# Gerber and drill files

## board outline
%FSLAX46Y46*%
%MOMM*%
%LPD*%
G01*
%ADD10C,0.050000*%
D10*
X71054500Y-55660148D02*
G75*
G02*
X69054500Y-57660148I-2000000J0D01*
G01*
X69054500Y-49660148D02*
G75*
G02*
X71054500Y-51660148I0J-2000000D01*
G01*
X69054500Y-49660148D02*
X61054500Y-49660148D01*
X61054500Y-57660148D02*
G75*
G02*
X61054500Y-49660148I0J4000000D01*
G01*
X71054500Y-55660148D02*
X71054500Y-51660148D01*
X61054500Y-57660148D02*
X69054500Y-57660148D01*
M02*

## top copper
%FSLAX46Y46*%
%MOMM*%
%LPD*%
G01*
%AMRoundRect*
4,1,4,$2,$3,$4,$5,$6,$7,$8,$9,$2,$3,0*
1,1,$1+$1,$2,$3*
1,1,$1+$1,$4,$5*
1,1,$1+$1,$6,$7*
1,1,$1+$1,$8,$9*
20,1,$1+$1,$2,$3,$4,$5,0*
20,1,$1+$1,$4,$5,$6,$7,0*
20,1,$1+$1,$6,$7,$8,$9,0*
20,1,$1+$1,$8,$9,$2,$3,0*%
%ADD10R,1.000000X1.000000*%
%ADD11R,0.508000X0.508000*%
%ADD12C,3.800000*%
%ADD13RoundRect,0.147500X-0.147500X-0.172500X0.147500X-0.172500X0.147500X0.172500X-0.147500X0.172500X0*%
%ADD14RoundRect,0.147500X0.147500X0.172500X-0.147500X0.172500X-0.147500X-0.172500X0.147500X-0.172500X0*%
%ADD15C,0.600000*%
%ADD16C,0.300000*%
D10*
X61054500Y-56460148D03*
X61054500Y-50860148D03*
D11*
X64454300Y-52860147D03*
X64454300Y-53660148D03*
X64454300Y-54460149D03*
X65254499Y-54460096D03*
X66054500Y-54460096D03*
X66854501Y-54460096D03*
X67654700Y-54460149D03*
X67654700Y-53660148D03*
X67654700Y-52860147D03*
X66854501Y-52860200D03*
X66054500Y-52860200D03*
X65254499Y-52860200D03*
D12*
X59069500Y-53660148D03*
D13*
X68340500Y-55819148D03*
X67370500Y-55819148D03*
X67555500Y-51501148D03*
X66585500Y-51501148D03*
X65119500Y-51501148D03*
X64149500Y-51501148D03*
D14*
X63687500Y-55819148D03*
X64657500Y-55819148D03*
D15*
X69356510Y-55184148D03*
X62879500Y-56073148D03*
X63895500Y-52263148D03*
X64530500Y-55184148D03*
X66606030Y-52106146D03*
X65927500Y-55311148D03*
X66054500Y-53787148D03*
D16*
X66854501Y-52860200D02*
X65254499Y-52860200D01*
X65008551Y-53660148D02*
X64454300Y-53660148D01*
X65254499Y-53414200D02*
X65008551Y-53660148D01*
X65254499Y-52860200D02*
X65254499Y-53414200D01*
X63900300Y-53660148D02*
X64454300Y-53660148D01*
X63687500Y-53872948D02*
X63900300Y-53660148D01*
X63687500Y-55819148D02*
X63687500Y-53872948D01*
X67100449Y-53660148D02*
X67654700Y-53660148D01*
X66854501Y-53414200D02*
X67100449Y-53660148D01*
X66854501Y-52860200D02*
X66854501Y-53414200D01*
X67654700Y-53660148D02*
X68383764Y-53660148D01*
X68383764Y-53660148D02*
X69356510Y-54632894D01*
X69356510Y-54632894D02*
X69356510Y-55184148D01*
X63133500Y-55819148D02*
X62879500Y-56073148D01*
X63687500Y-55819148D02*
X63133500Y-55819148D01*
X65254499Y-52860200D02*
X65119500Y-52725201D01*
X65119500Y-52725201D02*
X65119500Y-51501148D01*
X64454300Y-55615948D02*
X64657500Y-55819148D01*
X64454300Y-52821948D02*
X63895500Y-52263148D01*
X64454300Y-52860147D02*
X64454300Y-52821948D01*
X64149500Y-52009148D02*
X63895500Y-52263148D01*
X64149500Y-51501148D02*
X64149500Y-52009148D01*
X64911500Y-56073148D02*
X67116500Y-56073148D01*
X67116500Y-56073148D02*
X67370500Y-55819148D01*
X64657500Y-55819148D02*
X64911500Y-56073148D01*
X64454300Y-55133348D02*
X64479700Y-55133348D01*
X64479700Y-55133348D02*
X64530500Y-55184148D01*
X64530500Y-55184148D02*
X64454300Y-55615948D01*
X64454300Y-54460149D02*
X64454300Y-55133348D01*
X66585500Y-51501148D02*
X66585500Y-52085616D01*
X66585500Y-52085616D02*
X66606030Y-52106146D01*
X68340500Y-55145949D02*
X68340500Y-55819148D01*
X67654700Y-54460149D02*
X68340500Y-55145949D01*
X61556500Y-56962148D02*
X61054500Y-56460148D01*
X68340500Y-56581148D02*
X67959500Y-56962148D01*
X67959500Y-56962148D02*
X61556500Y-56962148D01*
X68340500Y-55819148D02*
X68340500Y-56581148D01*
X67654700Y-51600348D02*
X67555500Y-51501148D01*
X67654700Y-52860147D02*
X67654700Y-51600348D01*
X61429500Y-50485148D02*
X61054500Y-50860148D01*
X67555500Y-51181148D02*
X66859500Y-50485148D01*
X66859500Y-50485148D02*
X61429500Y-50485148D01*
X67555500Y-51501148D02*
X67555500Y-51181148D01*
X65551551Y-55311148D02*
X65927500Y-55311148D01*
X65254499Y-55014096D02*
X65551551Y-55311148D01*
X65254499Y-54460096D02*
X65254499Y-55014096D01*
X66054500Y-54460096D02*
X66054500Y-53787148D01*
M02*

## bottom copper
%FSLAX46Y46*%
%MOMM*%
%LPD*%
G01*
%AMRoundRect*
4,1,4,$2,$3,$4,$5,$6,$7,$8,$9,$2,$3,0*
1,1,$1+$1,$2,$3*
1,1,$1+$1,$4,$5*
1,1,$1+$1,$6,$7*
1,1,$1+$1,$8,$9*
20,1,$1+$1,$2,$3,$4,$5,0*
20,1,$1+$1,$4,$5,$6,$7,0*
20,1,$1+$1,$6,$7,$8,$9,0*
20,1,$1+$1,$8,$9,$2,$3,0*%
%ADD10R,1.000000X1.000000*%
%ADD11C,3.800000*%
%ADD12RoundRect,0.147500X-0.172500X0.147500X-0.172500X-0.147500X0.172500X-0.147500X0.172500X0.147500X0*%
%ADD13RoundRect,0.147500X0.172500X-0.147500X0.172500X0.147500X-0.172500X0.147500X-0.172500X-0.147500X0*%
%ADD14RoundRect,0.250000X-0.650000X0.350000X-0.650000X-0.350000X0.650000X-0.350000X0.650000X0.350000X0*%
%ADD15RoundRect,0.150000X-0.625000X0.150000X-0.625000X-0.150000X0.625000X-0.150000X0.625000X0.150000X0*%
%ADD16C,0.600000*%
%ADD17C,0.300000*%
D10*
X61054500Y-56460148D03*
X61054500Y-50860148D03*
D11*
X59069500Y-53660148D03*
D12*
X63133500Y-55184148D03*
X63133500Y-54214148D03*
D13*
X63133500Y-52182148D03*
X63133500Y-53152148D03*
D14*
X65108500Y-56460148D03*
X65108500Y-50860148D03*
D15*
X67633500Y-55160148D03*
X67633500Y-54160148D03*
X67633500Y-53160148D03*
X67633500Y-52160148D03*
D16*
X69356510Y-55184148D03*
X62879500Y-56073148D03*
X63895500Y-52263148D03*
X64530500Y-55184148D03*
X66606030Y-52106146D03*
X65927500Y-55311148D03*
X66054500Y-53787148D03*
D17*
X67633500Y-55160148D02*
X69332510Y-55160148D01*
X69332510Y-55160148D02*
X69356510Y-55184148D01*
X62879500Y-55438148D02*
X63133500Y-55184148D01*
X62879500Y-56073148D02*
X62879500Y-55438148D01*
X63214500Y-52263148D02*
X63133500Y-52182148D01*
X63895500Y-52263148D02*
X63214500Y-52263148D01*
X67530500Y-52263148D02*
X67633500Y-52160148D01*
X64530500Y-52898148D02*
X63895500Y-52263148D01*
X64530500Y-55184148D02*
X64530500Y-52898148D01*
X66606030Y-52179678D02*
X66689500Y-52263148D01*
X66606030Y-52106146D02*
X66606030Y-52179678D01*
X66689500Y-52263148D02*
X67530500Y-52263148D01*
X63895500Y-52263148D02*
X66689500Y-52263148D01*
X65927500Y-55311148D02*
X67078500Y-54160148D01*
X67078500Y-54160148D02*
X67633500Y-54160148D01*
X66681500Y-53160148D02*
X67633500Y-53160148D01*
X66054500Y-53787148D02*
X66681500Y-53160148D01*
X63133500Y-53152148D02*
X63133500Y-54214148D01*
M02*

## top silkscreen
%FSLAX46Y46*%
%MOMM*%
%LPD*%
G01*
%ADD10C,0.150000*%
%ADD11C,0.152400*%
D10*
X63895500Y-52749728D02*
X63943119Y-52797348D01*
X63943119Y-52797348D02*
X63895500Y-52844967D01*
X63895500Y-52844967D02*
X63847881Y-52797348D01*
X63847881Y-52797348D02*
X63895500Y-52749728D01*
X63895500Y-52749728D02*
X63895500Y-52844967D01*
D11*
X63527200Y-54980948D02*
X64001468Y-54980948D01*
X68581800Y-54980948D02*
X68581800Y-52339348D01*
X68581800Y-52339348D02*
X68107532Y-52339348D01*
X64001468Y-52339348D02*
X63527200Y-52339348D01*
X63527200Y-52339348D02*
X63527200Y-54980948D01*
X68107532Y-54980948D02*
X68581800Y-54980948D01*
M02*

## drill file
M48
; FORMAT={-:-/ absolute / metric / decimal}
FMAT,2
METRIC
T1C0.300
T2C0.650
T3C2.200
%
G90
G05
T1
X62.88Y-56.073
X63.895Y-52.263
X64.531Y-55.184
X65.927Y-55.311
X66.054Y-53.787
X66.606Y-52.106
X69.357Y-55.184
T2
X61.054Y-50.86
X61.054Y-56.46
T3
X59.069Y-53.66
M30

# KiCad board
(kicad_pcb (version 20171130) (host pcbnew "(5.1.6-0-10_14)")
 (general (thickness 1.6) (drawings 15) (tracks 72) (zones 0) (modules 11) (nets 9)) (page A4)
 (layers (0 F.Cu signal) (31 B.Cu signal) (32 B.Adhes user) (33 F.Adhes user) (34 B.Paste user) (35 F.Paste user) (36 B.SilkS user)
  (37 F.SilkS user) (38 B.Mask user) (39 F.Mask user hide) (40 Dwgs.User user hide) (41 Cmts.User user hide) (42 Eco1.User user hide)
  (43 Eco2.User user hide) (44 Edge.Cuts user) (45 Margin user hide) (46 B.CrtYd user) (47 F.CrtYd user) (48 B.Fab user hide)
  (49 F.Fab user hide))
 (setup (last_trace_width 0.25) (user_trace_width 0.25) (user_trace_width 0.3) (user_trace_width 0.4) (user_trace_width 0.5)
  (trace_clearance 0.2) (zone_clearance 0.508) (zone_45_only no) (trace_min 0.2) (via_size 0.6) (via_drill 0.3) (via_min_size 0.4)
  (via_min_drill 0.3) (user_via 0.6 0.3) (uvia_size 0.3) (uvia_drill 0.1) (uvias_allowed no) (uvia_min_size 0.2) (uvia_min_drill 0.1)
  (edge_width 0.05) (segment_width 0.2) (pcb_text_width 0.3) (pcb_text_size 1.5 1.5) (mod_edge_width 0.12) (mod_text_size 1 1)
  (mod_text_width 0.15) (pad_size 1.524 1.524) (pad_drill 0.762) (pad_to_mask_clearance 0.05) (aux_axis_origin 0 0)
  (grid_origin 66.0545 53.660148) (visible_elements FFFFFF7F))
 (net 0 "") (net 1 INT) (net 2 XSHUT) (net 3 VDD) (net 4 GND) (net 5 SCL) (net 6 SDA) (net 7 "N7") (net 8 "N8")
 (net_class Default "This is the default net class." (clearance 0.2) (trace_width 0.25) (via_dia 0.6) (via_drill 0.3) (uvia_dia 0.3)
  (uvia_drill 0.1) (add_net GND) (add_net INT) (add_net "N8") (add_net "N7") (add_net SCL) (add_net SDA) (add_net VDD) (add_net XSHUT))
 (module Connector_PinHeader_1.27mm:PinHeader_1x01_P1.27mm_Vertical (layer F.Cu) (at 61.0545 56.460148)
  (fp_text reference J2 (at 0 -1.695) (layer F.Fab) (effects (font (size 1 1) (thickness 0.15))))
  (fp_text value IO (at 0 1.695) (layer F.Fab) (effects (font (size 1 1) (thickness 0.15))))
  (pad 1 thru_hole rect (at 0 0) (size 1 1) (drill 0.65) (layers *.Cu *.Mask) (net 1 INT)))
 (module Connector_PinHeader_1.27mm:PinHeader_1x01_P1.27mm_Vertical (layer F.Cu) (at 61.0545 50.860148 270)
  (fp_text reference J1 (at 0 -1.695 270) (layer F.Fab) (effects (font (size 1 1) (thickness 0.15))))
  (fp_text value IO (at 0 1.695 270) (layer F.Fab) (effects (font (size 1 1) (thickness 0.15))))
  (pad 1 thru_hole rect (at 0 0 270) (size 1 1) (drill 0.65) (layers *.Cu *.Mask) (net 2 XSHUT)))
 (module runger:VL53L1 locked (layer F.Cu) (at 66.0545 53.660148)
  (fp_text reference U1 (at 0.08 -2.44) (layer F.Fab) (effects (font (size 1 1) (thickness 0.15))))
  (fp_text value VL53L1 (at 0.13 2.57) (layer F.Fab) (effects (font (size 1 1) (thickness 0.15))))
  (fp_line (start -2.5273 1.3208) (end -2.053032 1.3208) (layer F.SilkS) (width 0.1524))
  (fp_line (start 2.5273 1.3208) (end 2.5273 -1.3208) (layer F.SilkS) (width 0.1524))
  (fp_line (start 2.5273 -1.3208) (end 2.053032 -1.3208) (layer F.SilkS) (width 0.1524))
  (fp_line (start -2.053032 -1.3208) (end -2.5273 -1.3208) (layer F.SilkS) (width 0.1524))
  (fp_line (start -2.5273 -1.3208) (end -2.5273 1.3208) (layer F.SilkS) (width 0.1524))
  (fp_line (start 2.053032 1.3208) (end 2.5273 1.3208) (layer F.SilkS) (width 0.1524))
  (pad 1 smd rect (at -1.6002 -0.800001 90) (size 0.508 0.508) (layers F.Cu F.Paste F.Mask) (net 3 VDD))
  (pad 12 smd rect (at -1.6002 0 90) (size 0.508 0.508) (layers F.Cu F.Paste F.Mask) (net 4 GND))
  (pad 11 smd rect (at -1.6002 0.800001 90) (size 0.508 0.508) (layers F.Cu F.Paste F.Mask) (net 3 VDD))
  (pad 10 smd rect (at -0.800001 0.799948) (size 0.508 0.508) (layers F.Cu F.Paste F.Mask) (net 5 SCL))
  (pad 9 smd rect (at 0 0.799948) (size 0.508 0.508) (layers F.Cu F.Paste F.Mask) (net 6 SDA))
  (pad 8 smd rect (at 0.800001 0.799948) (size 0.508 0.508) (layers F.Cu F.Paste F.Mask) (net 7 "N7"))
  (pad 7 smd rect (at 1.6002 0.800001 90) (size 0.508 0.508) (layers F.Cu F.Paste F.Mask) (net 1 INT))
  (pad 6 smd rect (at 1.6002 0 90) (size 0.508 0.508) (layers F.Cu F.Paste F.Mask) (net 4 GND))
  (pad 5 smd rect (at 1.6002 -0.800001 90) (size 0.508 0.508) (layers F.Cu F.Paste F.Mask) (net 2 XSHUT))
  (pad 4 smd rect (at 0.800001 -0.799948) (size 0.508 0.508) (layers F.Cu F.Paste F.Mask) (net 4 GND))
  (pad 3 smd rect (at 0 -0.799948) (size 0.508 0.508) (layers F.Cu F.Paste F.Mask) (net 4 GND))
  (pad 2 smd rect (at -0.800001 -0.799948) (size 0.508 0.508) (layers F.Cu F.Paste F.Mask) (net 4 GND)))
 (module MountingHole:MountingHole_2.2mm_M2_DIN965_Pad (layer F.Cu) (at 59.0695 53.660148)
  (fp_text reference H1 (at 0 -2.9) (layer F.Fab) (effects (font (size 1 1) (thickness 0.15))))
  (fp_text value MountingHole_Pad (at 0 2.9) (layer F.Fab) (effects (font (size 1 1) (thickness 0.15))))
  (pad 1 thru_hole circle (at 0 0) (size 3.8 3.8) (drill 2.2) (layers *.Cu *.Mask)))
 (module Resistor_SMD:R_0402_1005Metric (layer B.Cu) (at 63.1335 54.699148 270)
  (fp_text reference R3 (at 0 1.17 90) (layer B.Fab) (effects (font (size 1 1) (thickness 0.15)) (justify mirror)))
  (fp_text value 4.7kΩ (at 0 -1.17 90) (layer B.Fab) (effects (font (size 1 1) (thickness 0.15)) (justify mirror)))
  (pad 2 smd roundrect (at 0.485 0 270) (size 0.59 0.64) (layers B.Cu B.Paste B.Mask) (roundrect_rratio 0.25) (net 4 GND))
  (pad 1 smd roundrect (at -0.485 0 270) (size 0.59 0.64) (layers B.Cu B.Paste B.Mask) (roundrect_rratio 0.25) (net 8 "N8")))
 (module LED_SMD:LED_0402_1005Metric (layer B.Cu) (at 63.1335 52.667148 90)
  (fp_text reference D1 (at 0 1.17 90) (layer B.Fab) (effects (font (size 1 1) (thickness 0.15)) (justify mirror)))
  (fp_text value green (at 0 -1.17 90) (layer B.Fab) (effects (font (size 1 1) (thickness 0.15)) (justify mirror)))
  (pad 2 smd roundrect (at 0.485 0 90) (size 0.59 0.64) (layers B.Cu B.Paste B.Mask) (roundrect_rratio 0.25) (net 3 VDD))
  (pad 1 smd roundrect (at -0.485 0 90) (size 0.59 0.64) (layers B.Cu B.Paste B.Mask) (roundrect_rratio 0.25) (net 8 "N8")))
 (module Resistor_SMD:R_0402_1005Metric (layer F.Cu) (at 67.8555 55.819148)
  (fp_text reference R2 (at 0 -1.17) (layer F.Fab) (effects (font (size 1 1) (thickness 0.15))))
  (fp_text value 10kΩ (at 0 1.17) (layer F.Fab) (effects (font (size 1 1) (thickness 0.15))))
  (pad 2 smd roundrect (at 0.485 0) (size 0.59 0.64) (layers F.Cu F.Paste F.Mask) (roundrect_rratio 0.25) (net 1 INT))
  (pad 1 smd roundrect (at -0.485 0) (size 0.59 0.64) (layers F.Cu F.Paste F.Mask) (roundrect_rratio 0.25) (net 3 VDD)))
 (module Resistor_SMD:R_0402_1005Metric (layer F.Cu) (at 67.0705 51.501148)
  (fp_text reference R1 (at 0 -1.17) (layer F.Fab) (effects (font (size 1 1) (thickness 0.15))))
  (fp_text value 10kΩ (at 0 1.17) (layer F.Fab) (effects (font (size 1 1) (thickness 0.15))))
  (pad 2 smd roundrect (at 0.485 0) (size 0.59 0.64) (layers F.Cu F.Paste F.Mask) (roundrect_rratio 0.25) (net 2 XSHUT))
  (pad 1 smd roundrect (at -0.485 0) (size 0.59 0.64) (layers F.Cu F.Paste F.Mask) (roundrect_rratio 0.25) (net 3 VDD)))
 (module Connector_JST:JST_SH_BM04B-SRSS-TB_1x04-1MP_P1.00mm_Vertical (layer B.Cu) (at 66.3085 53.660148 270)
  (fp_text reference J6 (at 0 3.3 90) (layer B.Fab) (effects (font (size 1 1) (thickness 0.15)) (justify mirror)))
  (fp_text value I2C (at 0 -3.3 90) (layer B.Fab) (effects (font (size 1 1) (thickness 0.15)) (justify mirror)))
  (pad MP smd roundrect (at 2.8 1.2 270) (size 1.2 1.8) (layers B.Cu B.Paste B.Mask) (roundrect_rratio 0.208333))
  (pad MP smd roundrect (at -2.8 1.2 270) (size 1.2 1.8) (layers B.Cu B.Paste B.Mask) (roundrect_rratio 0.208333))
  (pad 4 smd roundrect (at 1.5 -1.325 270) (size 0.6 1.55) (layers B.Cu B.Paste B.Mask) (roundrect_rratio 0.25) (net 4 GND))
  (pad 3 smd roundrect (at 0.5 -1.325 270) (size 0.6 1.55) (layers B.Cu B.Paste B.Mask) (roundrect_rratio 0.25) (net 5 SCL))
  (pad 2 smd roundrect (at -0.5 -1.325 270) (size 0.6 1.55) (layers B.Cu B.Paste B.Mask) (roundrect_rratio 0.25) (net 6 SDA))
  (pad 1 smd roundrect (at -1.5 -1.325 270) (size 0.6 1.55) (layers B.Cu B.Paste B.Mask) (roundrect_rratio 0.25) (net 3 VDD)))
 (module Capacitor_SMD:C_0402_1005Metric (layer F.Cu) (at 64.6345 51.501148)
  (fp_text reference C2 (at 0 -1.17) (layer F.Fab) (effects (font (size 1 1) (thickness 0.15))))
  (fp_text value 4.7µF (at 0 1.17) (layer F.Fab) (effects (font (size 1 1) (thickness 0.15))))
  (pad 2 smd roundrect (at 0.485 0) (size 0.59 0.64) (layers F.Cu F.Paste F.Mask) (roundrect_rratio 0.25) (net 4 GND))
  (pad 1 smd roundrect (at -0.485 0) (size 0.59 0.64) (layers F.Cu F.Paste F.Mask) (roundrect_rratio 0.25) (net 3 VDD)))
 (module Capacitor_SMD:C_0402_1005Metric (layer F.Cu) (at 64.1725 55.819148 180)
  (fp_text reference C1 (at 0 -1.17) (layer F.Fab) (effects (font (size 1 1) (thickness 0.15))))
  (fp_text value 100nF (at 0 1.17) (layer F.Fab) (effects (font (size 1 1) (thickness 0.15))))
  (pad 2 smd roundrect (at 0.485 0 180) (size 0.59 0.64) (layers F.Cu F.Paste F.Mask) (roundrect_rratio 0.25) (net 4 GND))
  (pad 1 smd roundrect (at -0.485 0 180) (size 0.59 0.64) (layers F.Cu F.Paste F.Mask) (roundrect_rratio 0.25) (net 3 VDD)))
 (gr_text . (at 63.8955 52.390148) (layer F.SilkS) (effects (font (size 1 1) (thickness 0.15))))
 (gr_arc (start 69.0545 55.660148) (end 69.0545 57.660148) (angle -90) (layer Edge.Cuts) (width 0.05))
 (gr_arc (start 69.0545 51.660148) (end 71.0545 51.660148) (angle -90) (layer Edge.Cuts) (width 0.05))
 (gr_line (start 69.0545 49.660148) (end 61.0545 49.660148) (layer Edge.Cuts) (width 0.05))
 (gr_arc (start 61.0545 53.660148) (end 61.0545 49.660148) (angle -180) (layer Edge.Cuts) (width 0.05))
 (gr_line (start 71.0545 55.660148) (end 71.0545 51.660148) (layer Edge.Cuts) (width 0.05))
 (gr_line (start 61.0545 57.660148) (end 69.0545 57.660148) (layer Edge.Cuts) (width 0.05))
 (segment (start 66.854501 52.8602) (end 65.254499 52.8602) (width 0.3) (layer F.Cu) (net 4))
 (segment (start 65.008551 53.660148) (end 64.4543 53.660148) (width 0.3) (layer F.Cu) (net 4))
 (segment (start 65.254499 53.4142) (end 65.008551 53.660148) (width 0.3) (layer F.Cu) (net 4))
 (segment (start 65.254499 52.8602) (end 65.254499 53.4142) (width 0.3) (layer F.Cu) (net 4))
 (segment (start 63.9003 53.660148) (end 64.4543 53.660148) (width 0.3) (layer F.Cu) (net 4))
 (segment (start 63.6875 53.872948) (end 63.9003 53.660148) (width 0.3) (layer F.Cu) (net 4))
 (segment (start 63.6875 55.819148) (end 63.6875 53.872948) (width 0.3) (layer F.Cu) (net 4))
 (segment (start 67.100449 53.660148) (end 67.6547 53.660148) (width 0.3) (layer F.Cu) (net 4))
 (segment (start 66.854501 53.4142) (end 67.100449 53.660148) (width 0.3) (layer F.Cu) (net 4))
 (segment (start 66.854501 52.8602) (end 66.854501 53.4142) (width 0.3) (layer F.Cu) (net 4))
 (via (at 69.35651 55.184148) (size 0.6) (drill 0.3) (layers F.Cu B.Cu) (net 4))
 (segment (start 67.6547 53.660148) (end 68.383764 53.660148) (width 0.3) (layer F.Cu) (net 4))
 (segment (start 68.383764 53.660148) (end 69.35651 54.632894) (width 0.3) (layer F.Cu) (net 4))
 (segment (start 67.6335 55.160148) (end 69.33251 55.160148) (width 0.3) (layer B.Cu) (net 4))
 (segment (start 69.35651 54.632894) (end 69.35651 55.184148) (width 0.3) (layer F.Cu) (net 4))
 (segment (start 69.33251 55.160148) (end 69.35651 55.184148) (width 0.3) (layer B.Cu) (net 4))
 (segment (start 63.1335 55.819148) (end 62.8795 56.073148) (width 0.3) (layer F.Cu) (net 4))
 (via (at 62.8795 56.073148) (size 0.6) (drill 0.3) (layers F.Cu B.Cu) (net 4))
 (segment (start 63.6875 55.819148) (end 63.1335 55.819148) (width 0.3) (layer F.Cu) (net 4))
 (segment (start 62.8795 55.438148) (end 63.1335 55.184148) (width 0.3) (layer B.Cu) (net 4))
 (segment (start 62.8795 56.073148) (end 62.8795 55.438148) (width 0.3) (layer B.Cu) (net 4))
 (segment (start 65.254499 52.8602) (end 65.1195 52.725201) (width 0.3) (layer F.Cu) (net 4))
 (segment (start 65.1195 52.725201) (end 65.1195 51.501148) (width 0.3) (layer F.Cu) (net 4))
 (segment (start 64.4543 55.615948) (end 64.6575 55.819148) (width 0.3) (layer F.Cu) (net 3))
 (via (at 63.8955 52.263148) (size 0.6) (drill 0.3) (layers F.Cu B.Cu) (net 3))
 (segment (start 64.4543 52.821948) (end 63.8955 52.263148) (width 0.3) (layer F.Cu) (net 3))
 (segment (start 64.4543 52.860147) (end 64.4543 52.821948) (width 0.3) (layer F.Cu) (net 3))
 (segment (start 63.2145 52.263148) (end 63.1335 52.182148) (width 0.3) (layer B.Cu) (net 3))
 (segment (start 63.8955 52.263148) (end 63.2145 52.263148) (width 0.3) (layer B.Cu) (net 3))
 (segment (start 64.1495 52.009148) (end 63.8955 52.263148) (width 0.3) (layer F.Cu) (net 3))
 (segment (start 64.1495 51.501148) (end 64.1495 52.009148) (width 0.3) (layer F.Cu) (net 3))
 (segment (start 67.5305 52.263148) (end 67.6335 52.160148) (width 0.3) (layer B.Cu) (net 3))
 (segment (start 64.9115 56.073148) (end 67.1165 56.073148) (width 0.3) (layer F.Cu) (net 3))
 (segment (start 67.1165 56.073148) (end 67.3705 55.819148) (width 0.3) (layer F.Cu) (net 3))
 (segment (start 64.6575 55.819148) (end 64.9115 56.073148) (width 0.3) (layer F.Cu) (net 3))
 (segment (start 64.4543 55.133348) (end 64.4797 55.133348) (width 0.3) (layer F.Cu) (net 3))
 (segment (start 64.4797 55.133348) (end 64.5305 55.184148) (width 0.3) (layer F.Cu) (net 3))
 (segment (start 64.5305 55.184148) (end 64.4543 55.615948) (width 0.3) (layer F.Cu) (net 3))
 (via (at 64.5305 55.184148) (size 0.6) (drill 0.3) (layers F.Cu B.Cu) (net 3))
 (segment (start 64.4543 54.460149) (end 64.4543 55.133348) (width 0.3) (layer F.Cu) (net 3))
 (segment (start 64.5305 52.898148) (end 63.8955 52.263148) (width 0.3) (layer B.Cu) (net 3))
 (segment (start 64.5305 55.184148) (end 64.5305 52.898148) (width 0.3) (layer B.Cu) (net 3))
 (via (at 66.60603 52.106146) (size 0.6) (drill 0.3) (layers F.Cu B.Cu) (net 3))
 (segment (start 66.5855 51.501148) (end 66.5855 52.085616) (width 0.3) (layer F.Cu) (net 3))
 (segment (start 66.5855 52.085616) (end 66.60603 52.106146) (width 0.3) (layer F.Cu) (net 3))
 (segment (start 66.60603 52.179678) (end 66.6895 52.263148) (width 0.3) (layer B.Cu) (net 3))
 (segment (start 66.60603 52.106146) (end 66.60603 52.179678) (width 0.3) (layer B.Cu) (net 3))
 (segment (start 66.6895 52.263148) (end 67.5305 52.263148) (width 0.3) (layer B.Cu) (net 3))
 (segment (start 63.8955 52.263148) (end 66.6895 52.263148) (width 0.3) (layer B.Cu) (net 3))
 (segment (start 68.3405 55.145949) (end 68.3405 55.819148) (width 0.3) (layer F.Cu) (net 1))
 (segment (start 67.6547 54.460149) (end 68.3405 55.145949) (width 0.3) (layer F.Cu) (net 1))
 (segment (start 61.5565 56.962148) (end 61.0545 56.460148) (width 0.3) (layer F.Cu) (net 1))
 (segment (start 68.3405 56.581148) (end 67.9595 56.962148) (width 0.3) (layer F.Cu) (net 1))
 (segment (start 67.9595 56.962148) (end 61.5565 56.962148) (width 0.3) (layer F.Cu) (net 1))
 (segment (start 68.3405 55.819148) (end 68.3405 56.581148) (width 0.3) (layer F.Cu) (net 1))
 (segment (start 67.6547 51.600348) (end 67.5555 51.501148) (width 0.3) (layer F.Cu) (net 2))
 (segment (start 67.6547 52.860147) (end 67.6547 51.600348) (width 0.3) (layer F.Cu) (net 2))
 (segment (start 61.4295 50.485148) (end 61.0545 50.860148) (width 0.3) (layer F.Cu) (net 2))
 (segment (start 67.5555 51.181148) (end 66.8595 50.485148) (width 0.3) (layer F.Cu) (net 2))
 (segment (start 66.8595 50.485148) (end 61.4295 50.485148) (width 0.3) (layer F.Cu) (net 2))
 (segment (start 67.5555 51.501148) (end 67.5555 51.181148) (width 0.3) (layer F.Cu) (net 2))
 (via (at 65.9275 55.311148) (size 0.6) (drill 0.3) (layers F.Cu B.Cu) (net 5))
 (segment (start 65.551551 55.311148) (end 65.9275 55.311148) (width 0.3) (layer F.Cu) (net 5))
 (segment (start 65.254499 55.014096) (end 65.551551 55.311148) (width 0.3) (layer F.Cu) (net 5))
 (segment (start 65.254499 54.460096) (end 65.254499 55.014096) (width 0.3) (layer F.Cu) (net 5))
 (segment (start 65.9275 55.311148) (end 67.0785 54.160148) (width 0.3) (layer B.Cu) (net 5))
 (segment (start 67.0785 54.160148) (end 67.6335 54.160148) (width 0.3) (layer B.Cu) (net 5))
 (segment (start 66.0545 54.460096) (end 66.0545 53.787148) (width 0.3) (layer F.Cu) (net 6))
 (via (at 66.0545 53.787148) (size 0.6) (drill 0.3) (layers F.Cu B.Cu) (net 6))
 (segment (start 66.6815 53.160148) (end 67.6335 53.160148) (width 0.3) (layer B.Cu) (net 6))
 (segment (start 66.0545 53.787148) (end 66.6815 53.160148) (width 0.3) (layer B.Cu) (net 6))
 (segment (start 63.1335 53.152148) (end 63.1335 54.214148) (width 0.3) (layer B.Cu) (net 8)))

